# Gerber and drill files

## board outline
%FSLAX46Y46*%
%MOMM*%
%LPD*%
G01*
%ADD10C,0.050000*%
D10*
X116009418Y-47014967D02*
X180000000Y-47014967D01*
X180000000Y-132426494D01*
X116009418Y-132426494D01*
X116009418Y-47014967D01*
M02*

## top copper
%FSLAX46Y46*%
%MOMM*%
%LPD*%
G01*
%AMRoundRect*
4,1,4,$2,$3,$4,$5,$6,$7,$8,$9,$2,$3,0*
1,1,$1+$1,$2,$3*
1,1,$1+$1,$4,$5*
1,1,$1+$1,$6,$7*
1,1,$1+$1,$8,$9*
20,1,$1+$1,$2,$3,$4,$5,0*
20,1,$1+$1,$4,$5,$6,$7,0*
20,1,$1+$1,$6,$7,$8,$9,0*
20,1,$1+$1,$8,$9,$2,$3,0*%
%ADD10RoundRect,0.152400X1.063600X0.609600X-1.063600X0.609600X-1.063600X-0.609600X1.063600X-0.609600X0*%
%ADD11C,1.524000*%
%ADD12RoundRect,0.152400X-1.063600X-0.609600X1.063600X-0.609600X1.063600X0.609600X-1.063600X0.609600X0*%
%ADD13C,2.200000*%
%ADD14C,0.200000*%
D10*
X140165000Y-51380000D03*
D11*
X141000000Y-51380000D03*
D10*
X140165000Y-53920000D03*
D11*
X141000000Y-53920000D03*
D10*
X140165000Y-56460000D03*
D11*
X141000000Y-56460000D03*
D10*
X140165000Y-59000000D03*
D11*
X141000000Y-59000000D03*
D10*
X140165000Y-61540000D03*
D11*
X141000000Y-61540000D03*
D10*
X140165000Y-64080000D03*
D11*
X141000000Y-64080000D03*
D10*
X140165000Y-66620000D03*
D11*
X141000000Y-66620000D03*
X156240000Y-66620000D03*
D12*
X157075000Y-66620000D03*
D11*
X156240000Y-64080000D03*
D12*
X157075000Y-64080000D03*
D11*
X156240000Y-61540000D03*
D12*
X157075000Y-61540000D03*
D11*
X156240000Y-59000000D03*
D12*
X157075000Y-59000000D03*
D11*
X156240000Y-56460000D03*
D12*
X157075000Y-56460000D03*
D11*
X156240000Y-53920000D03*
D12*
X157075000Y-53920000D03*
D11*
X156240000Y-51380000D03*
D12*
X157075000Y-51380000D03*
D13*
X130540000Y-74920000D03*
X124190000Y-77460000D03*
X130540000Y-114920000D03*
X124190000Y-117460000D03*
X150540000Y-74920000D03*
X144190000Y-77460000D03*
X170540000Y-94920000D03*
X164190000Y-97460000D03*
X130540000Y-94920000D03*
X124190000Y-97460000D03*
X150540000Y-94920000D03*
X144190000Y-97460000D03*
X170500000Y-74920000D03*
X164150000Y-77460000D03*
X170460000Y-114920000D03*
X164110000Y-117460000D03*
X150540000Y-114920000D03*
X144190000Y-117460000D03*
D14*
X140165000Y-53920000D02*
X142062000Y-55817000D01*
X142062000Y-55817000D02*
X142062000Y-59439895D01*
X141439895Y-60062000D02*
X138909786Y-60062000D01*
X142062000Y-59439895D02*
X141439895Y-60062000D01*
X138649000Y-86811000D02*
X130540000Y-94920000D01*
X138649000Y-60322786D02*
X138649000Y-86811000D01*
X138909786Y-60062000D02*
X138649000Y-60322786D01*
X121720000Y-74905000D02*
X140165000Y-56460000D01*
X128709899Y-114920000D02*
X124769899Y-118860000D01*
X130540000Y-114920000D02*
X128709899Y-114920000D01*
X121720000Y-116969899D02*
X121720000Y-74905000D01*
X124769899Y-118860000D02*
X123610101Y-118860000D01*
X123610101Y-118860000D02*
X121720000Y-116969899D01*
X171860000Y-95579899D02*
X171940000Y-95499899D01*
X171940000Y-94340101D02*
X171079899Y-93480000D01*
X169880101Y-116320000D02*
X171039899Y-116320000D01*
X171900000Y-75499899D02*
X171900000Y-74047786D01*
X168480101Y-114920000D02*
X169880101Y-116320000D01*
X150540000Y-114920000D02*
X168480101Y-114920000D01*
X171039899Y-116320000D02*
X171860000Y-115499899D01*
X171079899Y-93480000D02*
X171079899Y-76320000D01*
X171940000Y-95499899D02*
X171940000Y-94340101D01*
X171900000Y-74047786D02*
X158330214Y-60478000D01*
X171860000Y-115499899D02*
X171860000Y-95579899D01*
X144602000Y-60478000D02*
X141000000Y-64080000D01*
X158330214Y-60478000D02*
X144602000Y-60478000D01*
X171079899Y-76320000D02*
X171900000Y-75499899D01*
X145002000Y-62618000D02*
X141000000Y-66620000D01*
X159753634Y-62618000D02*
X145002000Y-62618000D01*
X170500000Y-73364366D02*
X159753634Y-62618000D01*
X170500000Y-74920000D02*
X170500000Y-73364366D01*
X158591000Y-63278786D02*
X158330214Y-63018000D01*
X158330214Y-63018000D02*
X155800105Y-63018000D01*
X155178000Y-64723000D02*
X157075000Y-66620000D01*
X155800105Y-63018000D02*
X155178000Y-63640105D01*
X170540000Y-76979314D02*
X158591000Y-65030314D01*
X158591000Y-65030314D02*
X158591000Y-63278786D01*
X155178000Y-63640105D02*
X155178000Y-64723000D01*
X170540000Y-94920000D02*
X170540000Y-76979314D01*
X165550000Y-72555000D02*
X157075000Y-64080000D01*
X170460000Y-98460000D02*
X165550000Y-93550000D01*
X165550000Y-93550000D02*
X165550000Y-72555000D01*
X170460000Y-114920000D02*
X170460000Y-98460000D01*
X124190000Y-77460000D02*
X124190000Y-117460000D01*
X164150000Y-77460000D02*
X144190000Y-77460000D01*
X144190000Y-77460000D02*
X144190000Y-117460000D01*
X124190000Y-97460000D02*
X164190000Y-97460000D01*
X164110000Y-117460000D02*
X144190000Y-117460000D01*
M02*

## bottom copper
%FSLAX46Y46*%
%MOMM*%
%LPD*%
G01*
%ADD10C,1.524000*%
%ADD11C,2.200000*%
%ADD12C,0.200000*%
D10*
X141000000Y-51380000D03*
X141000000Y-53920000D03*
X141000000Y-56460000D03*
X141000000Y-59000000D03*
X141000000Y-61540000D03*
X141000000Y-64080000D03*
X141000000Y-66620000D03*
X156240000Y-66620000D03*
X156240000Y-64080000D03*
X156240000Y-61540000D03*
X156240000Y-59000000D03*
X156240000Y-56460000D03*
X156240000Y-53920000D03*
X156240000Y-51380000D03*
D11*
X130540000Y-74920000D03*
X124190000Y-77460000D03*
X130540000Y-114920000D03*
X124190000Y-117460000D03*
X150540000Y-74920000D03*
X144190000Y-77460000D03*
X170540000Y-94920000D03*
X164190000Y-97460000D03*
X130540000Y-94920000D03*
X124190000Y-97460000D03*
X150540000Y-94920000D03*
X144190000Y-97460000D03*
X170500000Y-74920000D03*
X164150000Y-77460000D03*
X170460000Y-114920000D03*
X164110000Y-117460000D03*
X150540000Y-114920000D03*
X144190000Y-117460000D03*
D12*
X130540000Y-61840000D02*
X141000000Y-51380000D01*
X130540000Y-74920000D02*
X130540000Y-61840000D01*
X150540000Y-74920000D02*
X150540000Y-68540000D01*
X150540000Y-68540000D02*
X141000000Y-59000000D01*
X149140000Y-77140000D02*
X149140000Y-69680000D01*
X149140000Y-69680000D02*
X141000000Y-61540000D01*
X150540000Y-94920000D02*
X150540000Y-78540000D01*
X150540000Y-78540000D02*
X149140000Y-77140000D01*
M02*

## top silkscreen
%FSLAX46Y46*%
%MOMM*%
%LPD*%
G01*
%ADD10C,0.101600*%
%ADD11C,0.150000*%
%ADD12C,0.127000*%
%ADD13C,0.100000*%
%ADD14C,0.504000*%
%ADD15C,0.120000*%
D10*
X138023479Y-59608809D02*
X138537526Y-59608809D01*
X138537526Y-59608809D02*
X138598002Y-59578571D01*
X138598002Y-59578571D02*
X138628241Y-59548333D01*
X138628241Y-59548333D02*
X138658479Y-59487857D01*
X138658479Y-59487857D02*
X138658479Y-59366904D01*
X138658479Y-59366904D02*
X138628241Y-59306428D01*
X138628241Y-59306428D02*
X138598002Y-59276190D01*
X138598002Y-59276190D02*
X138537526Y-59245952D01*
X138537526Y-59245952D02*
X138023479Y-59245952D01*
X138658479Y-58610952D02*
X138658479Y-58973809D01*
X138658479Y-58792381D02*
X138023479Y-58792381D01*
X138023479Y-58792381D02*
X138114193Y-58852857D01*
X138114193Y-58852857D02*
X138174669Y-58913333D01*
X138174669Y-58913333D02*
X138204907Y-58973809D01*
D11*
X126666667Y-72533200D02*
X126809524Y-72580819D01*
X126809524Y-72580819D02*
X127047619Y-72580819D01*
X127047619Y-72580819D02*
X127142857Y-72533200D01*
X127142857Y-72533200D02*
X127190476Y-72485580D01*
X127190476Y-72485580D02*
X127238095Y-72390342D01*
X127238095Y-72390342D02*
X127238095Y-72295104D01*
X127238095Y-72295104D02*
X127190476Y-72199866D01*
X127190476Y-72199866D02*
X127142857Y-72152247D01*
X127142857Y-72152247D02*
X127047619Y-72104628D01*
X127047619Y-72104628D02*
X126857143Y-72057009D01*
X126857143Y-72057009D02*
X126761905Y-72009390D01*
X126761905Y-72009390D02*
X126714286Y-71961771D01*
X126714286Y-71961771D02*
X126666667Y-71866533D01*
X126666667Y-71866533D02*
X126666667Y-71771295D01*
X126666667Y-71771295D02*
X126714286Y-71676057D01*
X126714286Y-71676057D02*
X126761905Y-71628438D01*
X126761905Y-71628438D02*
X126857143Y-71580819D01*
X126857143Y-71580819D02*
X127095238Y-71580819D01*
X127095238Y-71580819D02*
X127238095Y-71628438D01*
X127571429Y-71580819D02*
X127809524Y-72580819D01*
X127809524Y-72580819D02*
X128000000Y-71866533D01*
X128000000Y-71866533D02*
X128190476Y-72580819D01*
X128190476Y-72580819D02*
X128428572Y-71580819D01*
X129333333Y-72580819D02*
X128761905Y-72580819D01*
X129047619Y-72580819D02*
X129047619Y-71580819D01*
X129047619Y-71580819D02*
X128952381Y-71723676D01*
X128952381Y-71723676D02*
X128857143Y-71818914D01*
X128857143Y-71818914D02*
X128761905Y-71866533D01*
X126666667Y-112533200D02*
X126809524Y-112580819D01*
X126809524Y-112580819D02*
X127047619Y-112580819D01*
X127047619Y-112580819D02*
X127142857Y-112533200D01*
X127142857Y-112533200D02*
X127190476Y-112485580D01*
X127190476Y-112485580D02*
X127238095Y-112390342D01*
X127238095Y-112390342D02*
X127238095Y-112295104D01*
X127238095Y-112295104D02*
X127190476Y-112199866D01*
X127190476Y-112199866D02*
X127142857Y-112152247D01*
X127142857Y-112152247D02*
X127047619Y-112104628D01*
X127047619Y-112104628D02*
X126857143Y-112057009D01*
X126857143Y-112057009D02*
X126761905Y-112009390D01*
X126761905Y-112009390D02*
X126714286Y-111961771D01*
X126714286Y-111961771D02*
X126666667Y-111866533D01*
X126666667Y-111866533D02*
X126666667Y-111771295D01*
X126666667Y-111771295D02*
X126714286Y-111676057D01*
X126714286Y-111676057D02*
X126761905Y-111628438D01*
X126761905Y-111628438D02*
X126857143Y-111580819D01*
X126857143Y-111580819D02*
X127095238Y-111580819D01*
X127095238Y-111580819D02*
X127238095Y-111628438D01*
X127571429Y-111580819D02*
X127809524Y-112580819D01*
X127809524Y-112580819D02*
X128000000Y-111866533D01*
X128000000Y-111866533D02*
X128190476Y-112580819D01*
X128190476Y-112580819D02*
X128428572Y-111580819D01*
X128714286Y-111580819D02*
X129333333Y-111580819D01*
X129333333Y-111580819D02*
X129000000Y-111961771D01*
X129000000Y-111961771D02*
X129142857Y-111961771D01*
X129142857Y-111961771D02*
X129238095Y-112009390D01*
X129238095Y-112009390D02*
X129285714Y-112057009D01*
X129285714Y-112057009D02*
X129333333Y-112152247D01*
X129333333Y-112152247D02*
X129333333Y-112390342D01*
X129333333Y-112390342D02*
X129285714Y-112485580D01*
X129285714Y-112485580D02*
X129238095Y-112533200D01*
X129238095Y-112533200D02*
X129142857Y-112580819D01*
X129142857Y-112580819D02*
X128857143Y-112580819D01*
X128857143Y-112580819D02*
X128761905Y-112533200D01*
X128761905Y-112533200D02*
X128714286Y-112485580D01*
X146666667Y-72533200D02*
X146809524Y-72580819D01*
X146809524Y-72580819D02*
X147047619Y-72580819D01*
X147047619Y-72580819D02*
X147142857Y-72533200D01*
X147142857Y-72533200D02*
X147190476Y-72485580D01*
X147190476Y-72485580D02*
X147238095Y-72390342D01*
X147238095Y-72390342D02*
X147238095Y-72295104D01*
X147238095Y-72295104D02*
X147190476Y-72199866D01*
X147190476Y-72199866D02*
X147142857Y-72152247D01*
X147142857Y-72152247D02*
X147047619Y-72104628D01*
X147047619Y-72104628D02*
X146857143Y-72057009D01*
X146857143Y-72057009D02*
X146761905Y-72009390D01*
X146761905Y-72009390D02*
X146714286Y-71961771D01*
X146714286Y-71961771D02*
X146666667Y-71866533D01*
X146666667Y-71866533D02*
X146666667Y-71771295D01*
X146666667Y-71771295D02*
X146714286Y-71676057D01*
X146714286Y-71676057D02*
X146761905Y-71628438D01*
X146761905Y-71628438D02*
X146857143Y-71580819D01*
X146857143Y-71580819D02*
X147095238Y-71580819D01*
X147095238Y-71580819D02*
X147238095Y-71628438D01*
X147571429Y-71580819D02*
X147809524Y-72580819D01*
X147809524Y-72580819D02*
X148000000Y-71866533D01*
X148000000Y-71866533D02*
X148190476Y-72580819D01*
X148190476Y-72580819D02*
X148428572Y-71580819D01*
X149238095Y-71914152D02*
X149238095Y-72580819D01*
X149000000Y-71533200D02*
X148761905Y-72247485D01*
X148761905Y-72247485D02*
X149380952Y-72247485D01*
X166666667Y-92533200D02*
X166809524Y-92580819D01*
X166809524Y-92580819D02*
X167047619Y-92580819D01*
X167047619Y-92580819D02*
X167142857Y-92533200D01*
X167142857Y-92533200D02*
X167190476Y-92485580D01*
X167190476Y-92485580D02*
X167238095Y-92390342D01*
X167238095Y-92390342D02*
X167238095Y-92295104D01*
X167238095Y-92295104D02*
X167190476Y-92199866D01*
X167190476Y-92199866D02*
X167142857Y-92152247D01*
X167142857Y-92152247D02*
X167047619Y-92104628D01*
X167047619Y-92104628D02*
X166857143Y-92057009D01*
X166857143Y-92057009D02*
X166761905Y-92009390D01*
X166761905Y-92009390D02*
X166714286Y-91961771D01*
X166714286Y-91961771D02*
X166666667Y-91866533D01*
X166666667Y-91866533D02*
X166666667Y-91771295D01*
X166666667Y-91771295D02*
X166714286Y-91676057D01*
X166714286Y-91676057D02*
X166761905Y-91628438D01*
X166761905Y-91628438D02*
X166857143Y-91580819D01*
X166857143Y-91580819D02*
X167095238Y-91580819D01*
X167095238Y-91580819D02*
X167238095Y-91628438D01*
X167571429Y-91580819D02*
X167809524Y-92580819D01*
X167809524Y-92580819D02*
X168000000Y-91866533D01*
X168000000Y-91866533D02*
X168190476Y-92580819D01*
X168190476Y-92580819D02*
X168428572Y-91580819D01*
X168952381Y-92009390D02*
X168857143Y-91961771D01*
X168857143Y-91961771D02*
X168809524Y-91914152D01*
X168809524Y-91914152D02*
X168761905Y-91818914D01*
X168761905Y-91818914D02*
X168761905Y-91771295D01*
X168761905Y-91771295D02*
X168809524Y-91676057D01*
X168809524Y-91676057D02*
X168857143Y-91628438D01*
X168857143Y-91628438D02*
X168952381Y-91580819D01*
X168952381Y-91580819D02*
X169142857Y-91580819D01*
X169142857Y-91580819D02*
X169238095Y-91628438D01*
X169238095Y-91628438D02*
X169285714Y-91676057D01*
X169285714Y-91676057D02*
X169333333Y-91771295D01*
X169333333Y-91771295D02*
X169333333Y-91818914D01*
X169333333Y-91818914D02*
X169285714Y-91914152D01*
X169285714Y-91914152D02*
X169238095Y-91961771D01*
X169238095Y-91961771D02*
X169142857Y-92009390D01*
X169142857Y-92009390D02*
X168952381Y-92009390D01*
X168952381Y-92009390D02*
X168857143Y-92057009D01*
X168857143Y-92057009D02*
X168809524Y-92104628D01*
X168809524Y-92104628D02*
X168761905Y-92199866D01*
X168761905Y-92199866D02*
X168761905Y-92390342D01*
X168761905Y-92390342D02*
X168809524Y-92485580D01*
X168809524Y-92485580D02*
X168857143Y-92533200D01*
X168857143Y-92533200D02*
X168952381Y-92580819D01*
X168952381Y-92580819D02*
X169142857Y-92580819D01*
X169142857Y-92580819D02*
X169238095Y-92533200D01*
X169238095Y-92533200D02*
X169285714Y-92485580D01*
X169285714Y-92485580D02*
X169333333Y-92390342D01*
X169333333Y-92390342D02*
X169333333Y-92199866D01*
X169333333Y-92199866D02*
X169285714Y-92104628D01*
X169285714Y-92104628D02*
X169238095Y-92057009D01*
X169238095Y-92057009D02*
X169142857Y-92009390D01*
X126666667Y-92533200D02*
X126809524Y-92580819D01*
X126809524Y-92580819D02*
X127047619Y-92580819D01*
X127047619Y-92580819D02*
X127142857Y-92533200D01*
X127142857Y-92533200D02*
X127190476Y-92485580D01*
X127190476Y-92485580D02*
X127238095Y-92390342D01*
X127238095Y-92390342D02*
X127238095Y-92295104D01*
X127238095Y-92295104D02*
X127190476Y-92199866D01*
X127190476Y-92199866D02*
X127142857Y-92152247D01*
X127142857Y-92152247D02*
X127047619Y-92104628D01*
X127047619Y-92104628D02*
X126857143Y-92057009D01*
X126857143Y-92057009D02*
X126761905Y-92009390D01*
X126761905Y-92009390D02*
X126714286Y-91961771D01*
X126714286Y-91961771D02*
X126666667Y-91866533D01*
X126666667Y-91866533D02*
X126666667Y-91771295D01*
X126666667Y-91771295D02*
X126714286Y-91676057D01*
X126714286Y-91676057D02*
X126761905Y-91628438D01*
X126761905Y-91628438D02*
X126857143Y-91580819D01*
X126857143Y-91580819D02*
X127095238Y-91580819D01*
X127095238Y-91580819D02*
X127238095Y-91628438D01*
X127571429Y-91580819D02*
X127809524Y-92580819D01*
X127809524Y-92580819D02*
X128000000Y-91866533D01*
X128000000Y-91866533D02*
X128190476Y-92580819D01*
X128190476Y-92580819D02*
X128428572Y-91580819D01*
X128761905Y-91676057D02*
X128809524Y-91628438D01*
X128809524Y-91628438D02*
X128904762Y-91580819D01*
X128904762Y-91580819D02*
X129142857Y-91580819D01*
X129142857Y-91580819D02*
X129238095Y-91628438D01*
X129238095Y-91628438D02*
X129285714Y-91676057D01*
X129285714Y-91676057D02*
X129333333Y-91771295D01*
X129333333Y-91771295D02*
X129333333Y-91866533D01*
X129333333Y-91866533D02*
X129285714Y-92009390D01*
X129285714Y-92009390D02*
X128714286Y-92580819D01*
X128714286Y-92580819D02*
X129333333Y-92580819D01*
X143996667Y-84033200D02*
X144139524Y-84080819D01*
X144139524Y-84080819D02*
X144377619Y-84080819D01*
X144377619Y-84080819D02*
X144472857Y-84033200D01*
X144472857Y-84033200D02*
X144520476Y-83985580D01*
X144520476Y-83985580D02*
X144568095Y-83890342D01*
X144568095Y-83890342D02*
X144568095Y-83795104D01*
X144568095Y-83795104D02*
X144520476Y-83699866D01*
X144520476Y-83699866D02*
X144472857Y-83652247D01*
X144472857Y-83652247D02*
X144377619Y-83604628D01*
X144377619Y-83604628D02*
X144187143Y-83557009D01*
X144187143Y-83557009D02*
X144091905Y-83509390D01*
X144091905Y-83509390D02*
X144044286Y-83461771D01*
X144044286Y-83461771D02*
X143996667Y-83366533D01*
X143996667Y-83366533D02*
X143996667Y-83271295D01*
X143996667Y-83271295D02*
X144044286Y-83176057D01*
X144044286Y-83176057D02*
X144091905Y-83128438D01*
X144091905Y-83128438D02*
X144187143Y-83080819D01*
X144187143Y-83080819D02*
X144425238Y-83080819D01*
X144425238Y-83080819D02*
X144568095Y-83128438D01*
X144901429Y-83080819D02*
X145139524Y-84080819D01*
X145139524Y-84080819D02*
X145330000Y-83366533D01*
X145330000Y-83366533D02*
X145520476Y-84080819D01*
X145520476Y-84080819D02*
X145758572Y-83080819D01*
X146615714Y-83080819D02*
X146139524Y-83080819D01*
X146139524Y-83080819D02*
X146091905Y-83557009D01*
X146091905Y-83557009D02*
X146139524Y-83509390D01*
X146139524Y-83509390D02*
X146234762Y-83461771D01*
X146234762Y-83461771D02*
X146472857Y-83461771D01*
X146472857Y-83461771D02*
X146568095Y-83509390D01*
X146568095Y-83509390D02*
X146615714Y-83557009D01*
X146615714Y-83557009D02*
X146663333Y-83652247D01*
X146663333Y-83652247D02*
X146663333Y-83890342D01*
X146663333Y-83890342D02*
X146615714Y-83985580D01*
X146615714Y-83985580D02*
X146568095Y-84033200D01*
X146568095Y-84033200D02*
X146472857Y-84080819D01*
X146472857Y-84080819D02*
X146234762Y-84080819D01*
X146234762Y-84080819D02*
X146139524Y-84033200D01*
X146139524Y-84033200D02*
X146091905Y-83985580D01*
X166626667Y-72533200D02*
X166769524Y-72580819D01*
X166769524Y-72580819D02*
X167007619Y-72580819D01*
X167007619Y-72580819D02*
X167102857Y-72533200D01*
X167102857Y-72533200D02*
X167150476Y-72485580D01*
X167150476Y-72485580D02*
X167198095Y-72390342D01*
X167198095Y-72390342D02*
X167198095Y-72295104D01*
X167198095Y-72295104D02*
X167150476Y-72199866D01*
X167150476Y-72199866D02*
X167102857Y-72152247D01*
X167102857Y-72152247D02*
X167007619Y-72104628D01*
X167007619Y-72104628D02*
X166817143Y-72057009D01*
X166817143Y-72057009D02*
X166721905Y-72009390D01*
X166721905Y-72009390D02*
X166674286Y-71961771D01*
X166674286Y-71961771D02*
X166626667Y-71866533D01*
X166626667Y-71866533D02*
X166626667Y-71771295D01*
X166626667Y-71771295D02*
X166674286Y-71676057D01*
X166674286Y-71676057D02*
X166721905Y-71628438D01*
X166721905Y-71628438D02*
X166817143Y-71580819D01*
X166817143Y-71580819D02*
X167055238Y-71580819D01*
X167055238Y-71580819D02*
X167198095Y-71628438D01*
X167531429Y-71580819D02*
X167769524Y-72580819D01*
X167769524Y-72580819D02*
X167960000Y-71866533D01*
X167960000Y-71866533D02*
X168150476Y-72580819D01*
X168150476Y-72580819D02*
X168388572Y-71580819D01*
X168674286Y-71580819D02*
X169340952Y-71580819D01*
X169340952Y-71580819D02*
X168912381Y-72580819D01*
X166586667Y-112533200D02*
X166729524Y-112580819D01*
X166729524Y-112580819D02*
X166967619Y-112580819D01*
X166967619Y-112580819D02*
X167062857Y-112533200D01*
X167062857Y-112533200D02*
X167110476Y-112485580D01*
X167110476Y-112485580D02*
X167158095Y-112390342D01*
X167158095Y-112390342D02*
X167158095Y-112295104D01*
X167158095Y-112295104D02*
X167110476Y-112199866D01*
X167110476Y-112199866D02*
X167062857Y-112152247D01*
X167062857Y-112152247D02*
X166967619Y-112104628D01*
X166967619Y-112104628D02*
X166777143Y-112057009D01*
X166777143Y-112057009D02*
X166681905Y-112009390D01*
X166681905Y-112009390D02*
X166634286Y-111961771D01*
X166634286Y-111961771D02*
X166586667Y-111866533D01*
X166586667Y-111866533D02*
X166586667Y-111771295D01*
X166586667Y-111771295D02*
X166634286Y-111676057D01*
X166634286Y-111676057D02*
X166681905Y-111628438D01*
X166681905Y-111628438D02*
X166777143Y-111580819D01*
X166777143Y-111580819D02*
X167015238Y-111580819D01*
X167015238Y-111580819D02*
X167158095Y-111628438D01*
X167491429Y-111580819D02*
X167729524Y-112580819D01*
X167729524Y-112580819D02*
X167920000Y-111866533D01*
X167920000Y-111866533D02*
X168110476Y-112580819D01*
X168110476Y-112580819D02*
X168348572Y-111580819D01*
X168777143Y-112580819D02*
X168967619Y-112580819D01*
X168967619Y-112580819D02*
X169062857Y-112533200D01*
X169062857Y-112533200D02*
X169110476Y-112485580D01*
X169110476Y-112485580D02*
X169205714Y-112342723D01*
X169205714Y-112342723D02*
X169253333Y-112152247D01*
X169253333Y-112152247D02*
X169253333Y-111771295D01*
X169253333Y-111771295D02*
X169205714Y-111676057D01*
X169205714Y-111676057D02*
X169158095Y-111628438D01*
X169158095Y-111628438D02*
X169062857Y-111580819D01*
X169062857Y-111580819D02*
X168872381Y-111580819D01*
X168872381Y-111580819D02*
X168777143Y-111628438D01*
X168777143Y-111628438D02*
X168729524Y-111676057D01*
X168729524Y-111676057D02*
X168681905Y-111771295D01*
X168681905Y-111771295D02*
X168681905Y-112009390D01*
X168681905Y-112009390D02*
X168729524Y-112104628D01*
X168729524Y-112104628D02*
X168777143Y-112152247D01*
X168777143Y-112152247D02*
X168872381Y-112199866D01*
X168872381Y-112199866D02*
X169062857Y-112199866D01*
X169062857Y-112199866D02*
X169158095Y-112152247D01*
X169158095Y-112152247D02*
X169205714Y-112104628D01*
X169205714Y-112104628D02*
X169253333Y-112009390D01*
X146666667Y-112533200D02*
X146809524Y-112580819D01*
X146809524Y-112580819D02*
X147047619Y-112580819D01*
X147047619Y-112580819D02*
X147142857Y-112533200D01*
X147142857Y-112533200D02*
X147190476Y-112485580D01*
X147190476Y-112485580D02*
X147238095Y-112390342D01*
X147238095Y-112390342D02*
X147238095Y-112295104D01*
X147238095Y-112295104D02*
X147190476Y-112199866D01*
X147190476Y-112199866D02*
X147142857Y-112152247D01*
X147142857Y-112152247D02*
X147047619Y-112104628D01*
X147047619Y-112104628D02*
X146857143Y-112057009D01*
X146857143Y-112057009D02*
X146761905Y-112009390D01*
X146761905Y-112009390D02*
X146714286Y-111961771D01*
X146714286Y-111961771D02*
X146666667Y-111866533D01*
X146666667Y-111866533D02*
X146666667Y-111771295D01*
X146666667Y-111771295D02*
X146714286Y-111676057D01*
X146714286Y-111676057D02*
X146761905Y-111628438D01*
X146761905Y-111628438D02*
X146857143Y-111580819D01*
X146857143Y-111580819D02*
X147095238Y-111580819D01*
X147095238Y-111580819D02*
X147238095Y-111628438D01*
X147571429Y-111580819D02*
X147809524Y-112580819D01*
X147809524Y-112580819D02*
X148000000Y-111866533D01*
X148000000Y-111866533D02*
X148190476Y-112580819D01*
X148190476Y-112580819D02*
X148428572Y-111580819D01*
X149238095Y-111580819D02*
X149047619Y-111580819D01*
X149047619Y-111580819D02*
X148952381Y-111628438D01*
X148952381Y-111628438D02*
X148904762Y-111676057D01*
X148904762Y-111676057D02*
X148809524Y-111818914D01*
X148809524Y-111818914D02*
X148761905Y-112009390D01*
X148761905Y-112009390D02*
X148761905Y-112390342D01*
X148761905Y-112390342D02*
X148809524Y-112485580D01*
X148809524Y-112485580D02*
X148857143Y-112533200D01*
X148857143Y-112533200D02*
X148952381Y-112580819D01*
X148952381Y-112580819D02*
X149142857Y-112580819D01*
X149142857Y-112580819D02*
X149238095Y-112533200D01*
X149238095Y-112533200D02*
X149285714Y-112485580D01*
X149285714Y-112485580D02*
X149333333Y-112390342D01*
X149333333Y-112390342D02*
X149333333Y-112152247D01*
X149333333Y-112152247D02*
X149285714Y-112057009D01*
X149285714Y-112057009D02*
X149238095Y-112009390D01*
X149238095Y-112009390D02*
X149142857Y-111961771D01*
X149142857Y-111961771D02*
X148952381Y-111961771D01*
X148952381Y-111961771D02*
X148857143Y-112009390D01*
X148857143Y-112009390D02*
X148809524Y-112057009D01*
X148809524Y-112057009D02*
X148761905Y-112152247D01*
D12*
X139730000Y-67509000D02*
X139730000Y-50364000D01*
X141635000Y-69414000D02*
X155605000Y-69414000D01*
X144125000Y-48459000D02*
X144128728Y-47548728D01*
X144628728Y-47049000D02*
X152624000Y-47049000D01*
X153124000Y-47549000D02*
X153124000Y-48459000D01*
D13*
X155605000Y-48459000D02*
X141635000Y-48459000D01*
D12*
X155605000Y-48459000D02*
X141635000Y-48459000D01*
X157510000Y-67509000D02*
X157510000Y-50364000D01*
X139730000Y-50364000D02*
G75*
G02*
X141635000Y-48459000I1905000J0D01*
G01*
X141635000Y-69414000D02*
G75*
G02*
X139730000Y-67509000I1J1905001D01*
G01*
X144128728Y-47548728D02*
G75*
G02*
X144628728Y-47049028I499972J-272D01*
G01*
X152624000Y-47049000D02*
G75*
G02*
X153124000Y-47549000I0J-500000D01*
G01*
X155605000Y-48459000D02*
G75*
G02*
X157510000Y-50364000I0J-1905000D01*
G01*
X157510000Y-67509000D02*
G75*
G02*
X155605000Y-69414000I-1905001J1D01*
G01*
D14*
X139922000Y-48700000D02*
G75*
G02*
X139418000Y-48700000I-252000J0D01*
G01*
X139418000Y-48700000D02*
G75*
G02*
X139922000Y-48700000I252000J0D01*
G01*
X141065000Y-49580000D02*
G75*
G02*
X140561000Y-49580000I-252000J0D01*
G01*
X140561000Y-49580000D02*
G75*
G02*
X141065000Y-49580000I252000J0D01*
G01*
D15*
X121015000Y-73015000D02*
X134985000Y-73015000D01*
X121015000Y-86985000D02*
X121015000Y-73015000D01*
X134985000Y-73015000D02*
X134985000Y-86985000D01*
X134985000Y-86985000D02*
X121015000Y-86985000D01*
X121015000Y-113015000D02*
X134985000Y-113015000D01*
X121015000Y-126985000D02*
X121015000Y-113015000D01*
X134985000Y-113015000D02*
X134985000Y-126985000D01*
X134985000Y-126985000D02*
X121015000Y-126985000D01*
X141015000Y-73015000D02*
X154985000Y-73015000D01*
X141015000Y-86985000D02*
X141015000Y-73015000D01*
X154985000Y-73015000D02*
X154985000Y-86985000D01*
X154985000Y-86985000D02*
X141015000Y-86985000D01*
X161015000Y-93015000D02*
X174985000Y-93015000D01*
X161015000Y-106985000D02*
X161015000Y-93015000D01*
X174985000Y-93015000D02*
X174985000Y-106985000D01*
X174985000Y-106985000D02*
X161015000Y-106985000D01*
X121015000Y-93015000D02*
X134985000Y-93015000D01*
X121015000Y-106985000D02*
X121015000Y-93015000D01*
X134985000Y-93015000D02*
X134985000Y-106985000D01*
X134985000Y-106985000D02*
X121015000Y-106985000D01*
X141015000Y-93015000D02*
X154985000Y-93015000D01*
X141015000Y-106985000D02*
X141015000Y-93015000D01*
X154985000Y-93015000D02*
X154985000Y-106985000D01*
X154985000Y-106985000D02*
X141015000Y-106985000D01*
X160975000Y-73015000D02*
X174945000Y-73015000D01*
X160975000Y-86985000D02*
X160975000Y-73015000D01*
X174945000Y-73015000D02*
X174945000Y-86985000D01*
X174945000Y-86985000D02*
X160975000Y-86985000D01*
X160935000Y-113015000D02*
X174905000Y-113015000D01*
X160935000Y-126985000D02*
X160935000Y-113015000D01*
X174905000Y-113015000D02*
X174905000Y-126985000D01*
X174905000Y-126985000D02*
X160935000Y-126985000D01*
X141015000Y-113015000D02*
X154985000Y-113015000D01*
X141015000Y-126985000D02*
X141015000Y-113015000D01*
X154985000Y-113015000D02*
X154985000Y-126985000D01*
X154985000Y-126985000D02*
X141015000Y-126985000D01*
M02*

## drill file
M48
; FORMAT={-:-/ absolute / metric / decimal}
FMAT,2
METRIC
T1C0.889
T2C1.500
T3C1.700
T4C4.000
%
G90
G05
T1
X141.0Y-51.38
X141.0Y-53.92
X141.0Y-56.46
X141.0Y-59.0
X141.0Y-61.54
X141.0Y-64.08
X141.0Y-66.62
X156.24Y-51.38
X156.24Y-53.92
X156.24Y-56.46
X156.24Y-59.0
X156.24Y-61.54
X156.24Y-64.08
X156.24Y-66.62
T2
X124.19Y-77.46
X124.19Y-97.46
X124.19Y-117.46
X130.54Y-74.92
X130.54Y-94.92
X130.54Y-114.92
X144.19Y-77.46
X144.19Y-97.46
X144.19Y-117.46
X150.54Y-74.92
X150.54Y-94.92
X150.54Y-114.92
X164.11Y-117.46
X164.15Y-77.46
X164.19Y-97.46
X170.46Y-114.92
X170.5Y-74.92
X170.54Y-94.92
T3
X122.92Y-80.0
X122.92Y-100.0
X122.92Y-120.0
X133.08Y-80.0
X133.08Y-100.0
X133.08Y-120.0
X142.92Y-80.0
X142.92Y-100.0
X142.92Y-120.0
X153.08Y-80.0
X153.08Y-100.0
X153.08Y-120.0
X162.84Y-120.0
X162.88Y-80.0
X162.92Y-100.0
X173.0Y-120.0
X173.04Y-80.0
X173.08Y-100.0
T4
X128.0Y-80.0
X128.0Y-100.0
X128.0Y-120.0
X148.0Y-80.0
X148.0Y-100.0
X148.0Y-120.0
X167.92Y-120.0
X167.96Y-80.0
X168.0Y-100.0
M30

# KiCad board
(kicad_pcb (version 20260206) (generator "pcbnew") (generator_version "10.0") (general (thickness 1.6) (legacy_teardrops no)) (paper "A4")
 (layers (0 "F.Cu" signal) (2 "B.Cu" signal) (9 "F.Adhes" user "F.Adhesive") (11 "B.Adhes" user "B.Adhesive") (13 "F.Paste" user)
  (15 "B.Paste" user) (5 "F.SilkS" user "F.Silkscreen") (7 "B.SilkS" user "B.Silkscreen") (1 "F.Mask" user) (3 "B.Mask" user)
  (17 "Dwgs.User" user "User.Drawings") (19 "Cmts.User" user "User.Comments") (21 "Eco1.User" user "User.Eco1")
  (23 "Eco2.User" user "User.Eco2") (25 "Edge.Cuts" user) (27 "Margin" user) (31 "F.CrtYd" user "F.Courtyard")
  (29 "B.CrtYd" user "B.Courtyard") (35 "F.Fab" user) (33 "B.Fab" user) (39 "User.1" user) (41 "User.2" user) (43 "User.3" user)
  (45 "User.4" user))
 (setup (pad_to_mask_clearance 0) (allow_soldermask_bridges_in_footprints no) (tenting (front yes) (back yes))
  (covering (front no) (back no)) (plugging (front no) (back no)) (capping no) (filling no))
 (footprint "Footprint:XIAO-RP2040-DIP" (layer "F.Cu") (at 148.62 59 90)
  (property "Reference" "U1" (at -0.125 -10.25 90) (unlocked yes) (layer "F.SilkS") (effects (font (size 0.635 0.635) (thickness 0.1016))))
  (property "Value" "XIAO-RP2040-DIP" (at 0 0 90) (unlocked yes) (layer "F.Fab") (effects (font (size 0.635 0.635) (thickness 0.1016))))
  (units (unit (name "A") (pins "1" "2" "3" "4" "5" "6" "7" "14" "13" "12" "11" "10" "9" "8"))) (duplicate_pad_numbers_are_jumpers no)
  (fp_line (start -8.509 -8.89) (end 8.636 -8.89) (stroke (width 0.127) (type solid)) (layer "F.SilkS"))
  (fp_line (start -10.414 -6.985) (end -10.414 6.985) (stroke (width 0.127) (type solid)) (layer "F.SilkS"))
  (fp_line (start 10.541 -4.495) (end 11.451272 -4.491272) (stroke (width 0.127) (type solid)) (layer "F.SilkS"))
  (fp_line (start 11.951 -3.991272) (end 11.951 4.004) (stroke (width 0.127) (type solid)) (layer "F.SilkS"))
  (fp_line (start 11.451 4.504) (end 10.541 4.504) (stroke (width 0.127) (type solid)) (layer "F.SilkS"))
  (fp_line (start 10.541 6.985) (end 10.541 -6.985) (stroke (width 0.1) (type solid)) (layer "F.SilkS"))
  (fp_line (start 10.541 6.985) (end 10.541 -6.985) (stroke (width 0.127) (type solid)) (layer "F.SilkS"))
  (fp_line (start -8.509 8.89) (end 8.636 8.89) (stroke (width 0.127) (type solid)) (layer "F.SilkS"))
  (fp_arc (start 8.636 -8.89) (mid 9.983038 -8.332038) (end 10.541 -6.985) (stroke (width 0.127) (type solid)) (layer "F.SilkS"))
  (fp_arc (start -10.414 -6.985) (mid -9.856038 -8.332038) (end -8.509 -8.89) (stroke (width 0.127) (type solid)) (layer "F.SilkS"))
  (fp_arc (start 11.451272 -4.491272) (mid 11.804644 -4.344724) (end 11.951 -3.991272) (stroke (width 0.127) (type default))
   (layer "F.SilkS"))
  (fp_arc (start 11.951 4.004) (mid 11.804553 4.357553) (end 11.451 4.504) (stroke (width 0.127) (type default)) (layer "F.SilkS"))
  (fp_arc (start 10.541 6.985) (mid 9.983038 8.332038) (end 8.636 8.89) (stroke (width 0.127) (type solid)) (layer "F.SilkS"))
  (fp_arc (start -8.509 8.89) (mid -9.856038 8.332038) (end -10.414 6.985) (stroke (width 0.127) (type solid)) (layer "F.SilkS"))
  (fp_circle (center 10.3 -8.95) (end 10.554 -8.95) (stroke (width 0.5) (type solid)) (fill yes) (layer "F.SilkS"))
  (fp_circle (center 9.42 -7.807) (end 9.674 -7.807) (stroke (width 0.5) (type solid)) (fill yes) (layer "F.SilkS"))
  (pad "1" smd roundrect (at 7.62 -8.455 180) (size 2.432 1.524) (layers "F.Cu" "F.Mask") (roundrect_rratio 0.1) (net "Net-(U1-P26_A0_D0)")
   (thermal_bridge_angle 45))
  (pad "1" thru_hole circle (at 7.62 -7.62 180) (size 1.524 1.524) (drill 0.889) (layers "*.Cu" "*.Mask") (remove_unused_layers no)
   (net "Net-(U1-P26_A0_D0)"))
  (pad "2" smd roundrect (at 5.08 -8.455 180) (size 2.432 1.524) (layers "F.Cu" "F.Mask") (roundrect_rratio 0.1) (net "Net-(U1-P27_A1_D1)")
   (thermal_bridge_angle 45))
  (pad "2" thru_hole circle (at 5.08 -7.62 180) (size 1.524 1.524) (drill 0.889) (layers "*.Cu" "*.Mask") (remove_unused_layers no)
   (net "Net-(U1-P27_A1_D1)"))
  (pad "3" smd roundrect (at 2.54 -8.455 180) (size 2.432 1.524) (layers "F.Cu" "F.Mask") (roundrect_rratio 0.1) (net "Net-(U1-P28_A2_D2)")
   (thermal_bridge_angle 45))
  (pad "3" thru_hole circle (at 2.54 -7.62 180) (size 1.524 1.524) (drill 0.889) (layers "*.Cu" "*.Mask") (remove_unused_layers no)
   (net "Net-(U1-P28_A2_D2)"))
  (pad "4" smd roundrect (at 0 -8.455 180) (size 2.432 1.524) (layers "F.Cu" "F.Mask") (roundrect_rratio 0.1) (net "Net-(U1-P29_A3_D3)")
   (thermal_bridge_angle 45))
  (pad "4" thru_hole circle (at 0 -7.62 180) (size 1.524 1.524) (drill 0.889) (layers "*.Cu" "*.Mask") (remove_unused_layers no)
   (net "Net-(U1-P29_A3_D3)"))
  (pad "5" smd roundrect (at -2.54 -8.455 180) (size 2.432 1.524) (layers "F.Cu" "F.Mask") (roundrect_rratio 0.1) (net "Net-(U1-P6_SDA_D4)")
   (thermal_bridge_angle 45))
  (pad "5" thru_hole circle (at -2.54 -7.62 180) (size 1.524 1.524) (drill 0.889) (layers "*.Cu" "*.Mask") (remove_unused_layers no)
   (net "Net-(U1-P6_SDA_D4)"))
  (pad "6" smd roundrect (at -5.08 -8.455 180) (size 2.432 1.524) (layers "F.Cu" "F.Mask") (roundrect_rratio 0.1) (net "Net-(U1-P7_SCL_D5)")
   (thermal_bridge_angle 45))
  (pad "6" thru_hole circle (at -5.08 -7.62 180) (size 1.524 1.524) (drill 0.889) (layers "*.Cu" "*.Mask") (remove_unused_layers no)
   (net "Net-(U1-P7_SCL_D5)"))
  (pad "7" smd roundrect (at -7.62 -8.455 180) (size 2.432 1.524) (layers "F.Cu" "F.Mask") (roundrect_rratio 0.1) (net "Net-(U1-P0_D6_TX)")
   (thermal_bridge_angle 45))
  (pad "7" thru_hole circle (at -7.62 -7.62 180) (size 1.524 1.524) (drill 0.889) (layers "*.Cu" "*.Mask") (remove_unused_layers no)
   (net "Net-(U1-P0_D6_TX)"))
  (pad "8" thru_hole circle (at -7.62 7.62) (size 1.524 1.524) (drill 0.889) (layers "*.Cu" "*.Mask") (remove_unused_layers no)
   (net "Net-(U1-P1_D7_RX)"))
  (pad "8" smd roundrect (at -7.62 8.455) (size 2.432 1.524) (layers "F.Cu" "F.Mask") (roundrect_rratio 0.1) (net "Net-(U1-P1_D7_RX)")
   (thermal_bridge_angle 45))
  (pad "9" thru_hole circle (at -5.08 7.62) (size 1.524 1.524) (drill 0.889) (layers "*.Cu" "*.Mask") (remove_unused_layers no)
   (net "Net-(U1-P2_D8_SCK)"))
  (pad "9" smd roundrect (at -5.08 8.455) (size 2.432 1.524) (layers "F.Cu" "F.Mask") (roundrect_rratio 0.1) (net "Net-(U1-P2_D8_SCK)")
   (thermal_bridge_angle 45))
  (pad "10" thru_hole circle (at -2.54 7.62) (size 1.524 1.524) (drill 0.889) (layers "*.Cu" "*.Mask") (remove_unused_layers no)
   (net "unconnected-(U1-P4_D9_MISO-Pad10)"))
  (pad "10" smd roundrect (at -2.54 8.455) (size 2.432 1.524) (layers "F.Cu" "F.Mask") (roundrect_rratio 0.1)
   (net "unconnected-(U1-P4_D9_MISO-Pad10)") (thermal_bridge_angle 45))
  (pad "11" thru_hole circle (at 0 7.62) (size 1.524 1.524) (drill 0.889) (layers "*.Cu" "*.Mask") (remove_unused_layers no)
   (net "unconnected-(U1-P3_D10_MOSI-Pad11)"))
  (pad "11" smd roundrect (at 0 8.455) (size 2.432 1.524) (layers "F.Cu" "F.Mask") (roundrect_rratio 0.1)
   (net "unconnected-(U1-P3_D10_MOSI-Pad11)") (thermal_bridge_angle 45))
  (pad "12" thru_hole circle (at 2.54 7.62) (size 1.524 1.524) (drill 0.889) (layers "*.Cu" "*.Mask") (remove_unused_layers no)
   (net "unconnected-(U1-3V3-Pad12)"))
  (pad "12" smd roundrect (at 2.54 8.455) (size 2.432 1.524) (layers "F.Cu" "F.Mask") (roundrect_rratio 0.1)
   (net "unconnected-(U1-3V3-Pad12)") (thermal_bridge_angle 45))
  (pad "13" thru_hole circle (at 5.08 7.62) (size 1.524 1.524) (drill 0.889) (layers "*.Cu" "*.Mask") (remove_unused_layers no)
   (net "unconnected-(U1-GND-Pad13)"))
  (pad "13" smd roundrect (at 5.08 8.455) (size 2.432 1.524) (layers "F.Cu" "F.Mask") (roundrect_rratio 0.1)
   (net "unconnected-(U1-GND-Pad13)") (thermal_bridge_angle 45))
  (pad "14" thru_hole circle (at 7.62 7.62) (size 1.524 1.524) (drill 0.889) (layers "*.Cu" "*.Mask") (remove_unused_layers no)
   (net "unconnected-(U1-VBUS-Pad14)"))
  (pad "14" smd roundrect (at 7.62 8.455) (size 2.432 1.524) (layers "F.Cu" "F.Mask") (roundrect_rratio 0.1)
   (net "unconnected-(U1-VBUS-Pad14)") (thermal_bridge_angle 45)))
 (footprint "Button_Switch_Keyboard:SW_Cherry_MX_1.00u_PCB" (layer "F.Cu") (at 130.54 74.92)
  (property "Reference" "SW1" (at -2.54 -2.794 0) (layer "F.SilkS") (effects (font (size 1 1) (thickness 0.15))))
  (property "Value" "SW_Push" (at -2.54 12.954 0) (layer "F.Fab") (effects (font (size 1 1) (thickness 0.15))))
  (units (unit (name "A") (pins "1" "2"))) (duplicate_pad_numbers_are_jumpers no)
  (fp_line (start -9.525 -1.905) (end 4.445 -1.905) (stroke (width 0.12) (type solid)) (layer "F.SilkS"))
  (fp_line (start -9.525 12.065) (end -9.525 -1.905) (stroke (width 0.12) (type solid)) (layer "F.SilkS"))
  (fp_line (start 4.445 -1.905) (end 4.445 12.065) (stroke (width 0.12) (type solid)) (layer "F.SilkS"))
  (fp_line (start 4.445 12.065) (end -9.525 12.065) (stroke (width 0.12) (type solid)) (layer "F.SilkS"))
  (pad "" np_thru_hole circle (at -7.62 5.08) (size 1.7 1.7) (drill 1.7) (layers "*.Cu" "*.Mask"))
  (pad "" np_thru_hole circle (at -2.54 5.08) (size 4 4) (drill 4) (layers "*.Cu" "*.Mask"))
  (pad "" np_thru_hole circle (at 2.54 5.08) (size 1.7 1.7) (drill 1.7) (layers "*.Cu" "*.Mask"))
  (pad "1" thru_hole circle (at 0 0) (size 2.2 2.2) (drill 1.5) (layers "*.Cu" "*.Mask") (remove_unused_layers no)
   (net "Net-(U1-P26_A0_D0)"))
  (pad "2" thru_hole circle (at -6.35 2.54) (size 2.2 2.2) (drill 1.5) (layers "*.Cu" "*.Mask") (remove_unused_layers no) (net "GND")))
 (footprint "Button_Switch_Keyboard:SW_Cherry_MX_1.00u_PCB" (layer "F.Cu") (at 130.54 114.92)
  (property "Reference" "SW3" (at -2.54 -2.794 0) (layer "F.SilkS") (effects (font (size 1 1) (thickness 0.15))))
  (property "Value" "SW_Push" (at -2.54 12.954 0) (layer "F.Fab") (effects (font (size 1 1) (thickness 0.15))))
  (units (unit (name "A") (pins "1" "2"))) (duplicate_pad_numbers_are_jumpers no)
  (fp_line (start -9.525 -1.905) (end 4.445 -1.905) (stroke (width 0.12) (type solid)) (layer "F.SilkS"))
  (fp_line (start -9.525 12.065) (end -9.525 -1.905) (stroke (width 0.12) (type solid)) (layer "F.SilkS"))
  (fp_line (start 4.445 -1.905) (end 4.445 12.065) (stroke (width 0.12) (type solid)) (layer "F.SilkS"))
  (fp_line (start 4.445 12.065) (end -9.525 12.065) (stroke (width 0.12) (type solid)) (layer "F.SilkS"))
  (pad "" np_thru_hole circle (at -7.62 5.08) (size 1.7 1.7) (drill 1.7) (layers "*.Cu" "*.Mask"))
  (pad "" np_thru_hole circle (at -2.54 5.08) (size 4 4) (drill 4) (layers "*.Cu" "*.Mask"))
  (pad "" np_thru_hole circle (at 2.54 5.08) (size 1.7 1.7) (drill 1.7) (layers "*.Cu" "*.Mask"))
  (pad "1" thru_hole circle (at 0 0) (size 2.2 2.2) (drill 1.5) (layers "*.Cu" "*.Mask") (remove_unused_layers no)
   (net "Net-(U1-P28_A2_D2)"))
  (pad "2" thru_hole circle (at -6.35 2.54) (size 2.2 2.2) (drill 1.5) (layers "*.Cu" "*.Mask") (remove_unused_layers no) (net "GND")))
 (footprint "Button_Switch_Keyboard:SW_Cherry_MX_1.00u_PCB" (layer "F.Cu") (at 150.54 74.92)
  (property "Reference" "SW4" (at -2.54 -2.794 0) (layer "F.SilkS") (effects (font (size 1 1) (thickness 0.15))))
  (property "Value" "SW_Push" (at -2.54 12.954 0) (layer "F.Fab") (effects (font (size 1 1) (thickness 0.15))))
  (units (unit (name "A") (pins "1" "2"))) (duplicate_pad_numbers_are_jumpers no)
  (fp_line (start -9.525 -1.905) (end 4.445 -1.905) (stroke (width 0.12) (type solid)) (layer "F.SilkS"))
  (fp_line (start -9.525 12.065) (end -9.525 -1.905) (stroke (width 0.12) (type solid)) (layer "F.SilkS"))
  (fp_line (start 4.445 -1.905) (end 4.445 12.065) (stroke (width 0.12) (type solid)) (layer "F.SilkS"))
  (fp_line (start 4.445 12.065) (end -9.525 12.065) (stroke (width 0.12) (type solid)) (layer "F.SilkS"))
  (pad "" np_thru_hole circle (at -7.62 5.08) (size 1.7 1.7) (drill 1.7) (layers "*.Cu" "*.Mask"))
  (pad "" np_thru_hole circle (at -2.54 5.08) (size 4 4) (drill 4) (layers "*.Cu" "*.Mask"))
  (pad "" np_thru_hole circle (at 2.54 5.08) (size 1.7 1.7) (drill 1.7) (layers "*.Cu" "*.Mask"))
  (pad "1" thru_hole circle (at 0 0) (size 2.2 2.2) (drill 1.5) (layers "*.Cu" "*.Mask") (remove_unused_layers no)
   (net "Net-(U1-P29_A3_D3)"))
  (pad "2" thru_hole circle (at -6.35 2.54) (size 2.2 2.2) (drill 1.5) (layers "*.Cu" "*.Mask") (remove_unused_layers no) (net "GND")))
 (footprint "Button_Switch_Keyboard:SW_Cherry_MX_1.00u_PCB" (layer "F.Cu") (at 170.54 94.92)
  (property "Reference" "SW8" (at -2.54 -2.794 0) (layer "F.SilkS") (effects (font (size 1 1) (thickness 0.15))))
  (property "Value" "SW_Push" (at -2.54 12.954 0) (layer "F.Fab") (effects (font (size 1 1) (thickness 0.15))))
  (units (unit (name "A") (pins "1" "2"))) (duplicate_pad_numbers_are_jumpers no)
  (fp_line (start -9.525 -1.905) (end 4.445 -1.905) (stroke (width 0.12) (type solid)) (layer "F.SilkS"))
  (fp_line (start -9.525 12.065) (end -9.525 -1.905) (stroke (width 0.12) (type solid)) (layer "F.SilkS"))
  (fp_line (start 4.445 -1.905) (end 4.445 12.065) (stroke (width 0.12) (type solid)) (layer "F.SilkS"))
  (fp_line (start 4.445 12.065) (end -9.525 12.065) (stroke (width 0.12) (type solid)) (layer "F.SilkS"))
  (pad "" np_thru_hole circle (at -7.62 5.08) (size 1.7 1.7) (drill 1.7) (layers "*.Cu" "*.Mask"))
  (pad "" np_thru_hole circle (at -2.54 5.08) (size 4 4) (drill 4) (layers "*.Cu" "*.Mask"))
  (pad "" np_thru_hole circle (at 2.54 5.08) (size 1.7 1.7) (drill 1.7) (layers "*.Cu" "*.Mask"))
  (pad "1" thru_hole circle (at 0 0) (size 2.2 2.2) (drill 1.5) (layers "*.Cu" "*.Mask") (remove_unused_layers no) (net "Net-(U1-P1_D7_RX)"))
  (pad "2" thru_hole circle (at -6.35 2.54) (size 2.2 2.2) (drill 1.5) (layers "*.Cu" "*.Mask") (remove_unused_layers no) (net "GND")))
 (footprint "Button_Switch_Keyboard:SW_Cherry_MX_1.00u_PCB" (layer "F.Cu") (at 130.54 94.92)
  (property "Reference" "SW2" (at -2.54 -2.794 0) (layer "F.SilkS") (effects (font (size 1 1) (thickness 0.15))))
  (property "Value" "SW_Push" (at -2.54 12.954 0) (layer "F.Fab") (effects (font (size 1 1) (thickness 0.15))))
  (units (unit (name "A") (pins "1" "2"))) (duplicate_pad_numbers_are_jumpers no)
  (fp_line (start -9.525 -1.905) (end 4.445 -1.905) (stroke (width 0.12) (type solid)) (layer "F.SilkS"))
  (fp_line (start -9.525 12.065) (end -9.525 -1.905) (stroke (width 0.12) (type solid)) (layer "F.SilkS"))
  (fp_line (start 4.445 -1.905) (end 4.445 12.065) (stroke (width 0.12) (type solid)) (layer "F.SilkS"))
  (fp_line (start 4.445 12.065) (end -9.525 12.065) (stroke (width 0.12) (type solid)) (layer "F.SilkS"))
  (pad "" np_thru_hole circle (at -7.62 5.08) (size 1.7 1.7) (drill 1.7) (layers "*.Cu" "*.Mask"))
  (pad "" np_thru_hole circle (at -2.54 5.08) (size 4 4) (drill 4) (layers "*.Cu" "*.Mask"))
  (pad "" np_thru_hole circle (at 2.54 5.08) (size 1.7 1.7) (drill 1.7) (layers "*.Cu" "*.Mask"))
  (pad "1" thru_hole circle (at 0 0) (size 2.2 2.2) (drill 1.5) (layers "*.Cu" "*.Mask") (remove_unused_layers no)
   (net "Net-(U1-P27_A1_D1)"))
  (pad "2" thru_hole circle (at -6.35 2.54) (size 2.2 2.2) (drill 1.5) (layers "*.Cu" "*.Mask") (remove_unused_layers no) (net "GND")))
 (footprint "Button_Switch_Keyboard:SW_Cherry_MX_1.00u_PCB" (layer "F.Cu") (at 150.54 94.92)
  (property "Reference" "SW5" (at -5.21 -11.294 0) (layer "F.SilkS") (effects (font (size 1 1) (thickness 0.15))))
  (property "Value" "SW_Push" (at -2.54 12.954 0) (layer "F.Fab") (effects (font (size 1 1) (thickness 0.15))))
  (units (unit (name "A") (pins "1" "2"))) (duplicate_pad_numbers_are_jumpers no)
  (fp_line (start -9.525 -1.905) (end 4.445 -1.905) (stroke (width 0.12) (type solid)) (layer "F.SilkS"))
  (fp_line (start -9.525 12.065) (end -9.525 -1.905) (stroke (width 0.12) (type solid)) (layer "F.SilkS"))
  (fp_line (start 4.445 -1.905) (end 4.445 12.065) (stroke (width 0.12) (type solid)) (layer "F.SilkS"))
  (fp_line (start 4.445 12.065) (end -9.525 12.065) (stroke (width 0.12) (type solid)) (layer "F.SilkS"))
  (pad "" np_thru_hole circle (at -7.62 5.08) (size 1.7 1.7) (drill 1.7) (layers "*.Cu" "*.Mask"))
  (pad "" np_thru_hole circle (at -2.54 5.08) (size 4 4) (drill 4) (layers "*.Cu" "*.Mask"))
  (pad "" np_thru_hole circle (at 2.54 5.08) (size 1.7 1.7) (drill 1.7) (layers "*.Cu" "*.Mask"))
  (pad "1" thru_hole circle (at 0 0) (size 2.2 2.2) (drill 1.5) (layers "*.Cu" "*.Mask") (remove_unused_layers no)
   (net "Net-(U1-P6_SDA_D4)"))
  (pad "2" thru_hole circle (at -6.35 2.54) (size 2.2 2.2) (drill 1.5) (layers "*.Cu" "*.Mask") (remove_unused_layers no) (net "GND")))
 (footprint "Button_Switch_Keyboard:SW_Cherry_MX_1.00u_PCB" (layer "F.Cu") (at 170.5 74.92)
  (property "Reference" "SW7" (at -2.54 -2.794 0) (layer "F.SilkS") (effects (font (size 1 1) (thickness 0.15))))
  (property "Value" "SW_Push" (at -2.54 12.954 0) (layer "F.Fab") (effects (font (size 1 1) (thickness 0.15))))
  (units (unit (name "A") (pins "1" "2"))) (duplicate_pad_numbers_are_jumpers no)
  (fp_line (start -9.525 -1.905) (end 4.445 -1.905) (stroke (width 0.12) (type solid)) (layer "F.SilkS"))
  (fp_line (start -9.525 12.065) (end -9.525 -1.905) (stroke (width 0.12) (type solid)) (layer "F.SilkS"))
  (fp_line (start 4.445 -1.905) (end 4.445 12.065) (stroke (width 0.12) (type solid)) (layer "F.SilkS"))
  (fp_line (start 4.445 12.065) (end -9.525 12.065) (stroke (width 0.12) (type solid)) (layer "F.SilkS"))
  (pad "" np_thru_hole circle (at -7.62 5.08) (size 1.7 1.7) (drill 1.7) (layers "*.Cu" "*.Mask"))
  (pad "" np_thru_hole circle (at -2.54 5.08) (size 4 4) (drill 4) (layers "*.Cu" "*.Mask"))
  (pad "" np_thru_hole circle (at 2.54 5.08) (size 1.7 1.7) (drill 1.7) (layers "*.Cu" "*.Mask"))
  (pad "1" thru_hole circle (at 0 0) (size 2.2 2.2) (drill 1.5) (layers "*.Cu" "*.Mask") (remove_unused_layers no) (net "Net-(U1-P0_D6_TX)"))
  (pad "2" thru_hole circle (at -6.35 2.54) (size 2.2 2.2) (drill 1.5) (layers "*.Cu" "*.Mask") (remove_unused_layers no) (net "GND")))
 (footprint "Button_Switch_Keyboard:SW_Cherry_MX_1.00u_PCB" (layer "F.Cu") (at 170.46 114.92)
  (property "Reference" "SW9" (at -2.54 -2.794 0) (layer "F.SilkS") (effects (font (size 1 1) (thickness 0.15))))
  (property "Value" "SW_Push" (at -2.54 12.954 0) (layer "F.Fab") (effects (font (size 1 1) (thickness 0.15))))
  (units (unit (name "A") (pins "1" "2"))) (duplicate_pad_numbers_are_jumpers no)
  (fp_line (start -9.525 -1.905) (end 4.445 -1.905) (stroke (width 0.12) (type solid)) (layer "F.SilkS"))
  (fp_line (start -9.525 12.065) (end -9.525 -1.905) (stroke (width 0.12) (type solid)) (layer "F.SilkS"))
  (fp_line (start 4.445 -1.905) (end 4.445 12.065) (stroke (width 0.12) (type solid)) (layer "F.SilkS"))
  (fp_line (start 4.445 12.065) (end -9.525 12.065) (stroke (width 0.12) (type solid)) (layer "F.SilkS"))
  (pad "" np_thru_hole circle (at -7.62 5.08) (size 1.7 1.7) (drill 1.7) (layers "*.Cu" "*.Mask"))
  (pad "" np_thru_hole circle (at -2.54 5.08) (size 4 4) (drill 4) (layers "*.Cu" "*.Mask"))
  (pad "" np_thru_hole circle (at 2.54 5.08) (size 1.7 1.7) (drill 1.7) (layers "*.Cu" "*.Mask"))
  (pad "1" thru_hole circle (at 0 0) (size 2.2 2.2) (drill 1.5) (layers "*.Cu" "*.Mask") (remove_unused_layers no)
   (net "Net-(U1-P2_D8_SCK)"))
  (pad "2" thru_hole circle (at -6.35 2.54) (size 2.2 2.2) (drill 1.5) (layers "*.Cu" "*.Mask") (remove_unused_layers no) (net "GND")))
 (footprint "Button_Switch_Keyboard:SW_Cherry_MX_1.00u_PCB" (layer "F.Cu") (at 150.54 114.92)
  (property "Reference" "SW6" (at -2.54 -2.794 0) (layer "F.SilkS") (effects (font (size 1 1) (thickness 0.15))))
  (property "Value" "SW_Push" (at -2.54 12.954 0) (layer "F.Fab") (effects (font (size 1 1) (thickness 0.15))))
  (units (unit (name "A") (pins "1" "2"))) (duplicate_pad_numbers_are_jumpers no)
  (fp_line (start -9.525 -1.905) (end 4.445 -1.905) (stroke (width 0.12) (type solid)) (layer "F.SilkS"))
  (fp_line (start -9.525 12.065) (end -9.525 -1.905) (stroke (width 0.12) (type solid)) (layer "F.SilkS"))
  (fp_line (start 4.445 -1.905) (end 4.445 12.065) (stroke (width 0.12) (type solid)) (layer "F.SilkS"))
  (fp_line (start 4.445 12.065) (end -9.525 12.065) (stroke (width 0.12) (type solid)) (layer "F.SilkS"))
  (pad "" np_thru_hole circle (at -7.62 5.08) (size 1.7 1.7) (drill 1.7) (layers "*.Cu" "*.Mask"))
  (pad "" np_thru_hole circle (at -2.54 5.08) (size 4 4) (drill 4) (layers "*.Cu" "*.Mask"))
  (pad "" np_thru_hole circle (at 2.54 5.08) (size 1.7 1.7) (drill 1.7) (layers "*.Cu" "*.Mask"))
  (pad "1" thru_hole circle (at 0 0) (size 2.2 2.2) (drill 1.5) (layers "*.Cu" "*.Mask") (remove_unused_layers no)
   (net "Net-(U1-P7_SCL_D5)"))
  (pad "2" thru_hole circle (at -6.35 2.54) (size 2.2 2.2) (drill 1.5) (layers "*.Cu" "*.Mask") (remove_unused_layers no) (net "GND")))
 (gr_rect (start 116.009418 47.014967) (end 180 132.426494) (stroke (width 0.05) (type default)) (fill no) (layer "Edge.Cuts"))
 (segment (start 130.54 61.84) (end 141 51.38) (width 0.2) (layer "B.Cu") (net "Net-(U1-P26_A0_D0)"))
 (segment (start 130.54 74.92) (end 130.54 61.84) (width 0.2) (layer "B.Cu") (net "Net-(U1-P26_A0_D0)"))
 (segment (start 140.165 53.92) (end 142.062 55.817) (width 0.2) (layer "F.Cu") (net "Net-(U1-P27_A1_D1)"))
 (segment (start 142.062 55.817) (end 142.062 59.439895) (width 0.2) (layer "F.Cu") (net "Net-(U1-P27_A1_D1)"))
 (segment (start 141.439895 60.062) (end 138.909786 60.062) (width 0.2) (layer "F.Cu") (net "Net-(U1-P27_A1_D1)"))
 (segment (start 142.062 59.439895) (end 141.439895 60.062) (width 0.2) (layer "F.Cu") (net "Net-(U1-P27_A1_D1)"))
 (segment (start 138.649 86.811) (end 130.54 94.92) (width 0.2) (layer "F.Cu") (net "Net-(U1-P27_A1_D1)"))
 (segment (start 138.649 60.322786) (end 138.649 86.811) (width 0.2) (layer "F.Cu") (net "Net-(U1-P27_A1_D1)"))
 (segment (start 138.909786 60.062) (end 138.649 60.322786) (width 0.2) (layer "F.Cu") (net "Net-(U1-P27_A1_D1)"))
 (segment (start 121.72 74.905) (end 140.165 56.46) (width 0.2) (layer "F.Cu") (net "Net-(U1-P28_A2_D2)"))
 (segment (start 128.709899 114.92) (end 124.769899 118.86) (width 0.2) (layer "F.Cu") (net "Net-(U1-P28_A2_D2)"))
 (segment (start 130.54 114.92) (end 128.709899 114.92) (width 0.2) (layer "F.Cu") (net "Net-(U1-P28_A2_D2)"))
 (segment (start 121.72 116.969899) (end 121.72 74.905) (width 0.2) (layer "F.Cu") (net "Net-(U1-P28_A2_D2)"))
 (segment (start 124.769899 118.86) (end 123.610101 118.86) (width 0.2) (layer "F.Cu") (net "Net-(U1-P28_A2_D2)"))
 (segment (start 123.610101 118.86) (end 121.72 116.969899) (width 0.2) (layer "F.Cu") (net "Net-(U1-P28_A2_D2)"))
 (segment (start 150.54 74.92) (end 150.54 68.54) (width 0.2) (layer "B.Cu") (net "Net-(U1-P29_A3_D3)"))
 (segment (start 150.54 68.54) (end 141 59) (width 0.2) (layer "B.Cu") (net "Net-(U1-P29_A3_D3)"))
 (segment (start 149.14 77.14) (end 149.14 69.68) (width 0.2) (layer "B.Cu") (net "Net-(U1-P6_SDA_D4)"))
 (segment (start 149.14 69.68) (end 141 61.54) (width 0.2) (layer "B.Cu") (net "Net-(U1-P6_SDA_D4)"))
 (segment (start 150.54 94.92) (end 150.54 78.54) (width 0.2) (layer "B.Cu") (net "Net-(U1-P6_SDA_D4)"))
 (segment (start 150.54 78.54) (end 149.14 77.14) (width 0.2) (layer "B.Cu") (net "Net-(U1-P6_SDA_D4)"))
 (segment (start 171.86 95.579899) (end 171.94 95.499899) (width 0.2) (layer "F.Cu") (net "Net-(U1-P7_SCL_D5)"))
 (segment (start 171.94 94.340101) (end 171.079899 93.48) (width 0.2) (layer "F.Cu") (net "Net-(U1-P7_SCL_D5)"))
 (segment (start 169.880101 116.32) (end 171.039899 116.32) (width 0.2) (layer "F.Cu") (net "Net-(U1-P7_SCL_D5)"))
 (segment (start 171.9 75.499899) (end 171.9 74.047786) (width 0.2) (layer "F.Cu") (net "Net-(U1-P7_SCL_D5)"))
 (segment (start 168.480101 114.92) (end 169.880101 116.32) (width 0.2) (layer "F.Cu") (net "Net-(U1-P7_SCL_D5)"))
 (segment (start 150.54 114.92) (end 168.480101 114.92) (width 0.2) (layer "F.Cu") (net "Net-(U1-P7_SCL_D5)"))
 (segment (start 171.039899 116.32) (end 171.86 115.499899) (width 0.2) (layer "F.Cu") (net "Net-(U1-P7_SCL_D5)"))
 (segment (start 171.079899 93.48) (end 171.079899 76.32) (width 0.2) (layer "F.Cu") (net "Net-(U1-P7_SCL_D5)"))
 (segment (start 171.94 95.499899) (end 171.94 94.340101) (width 0.2) (layer "F.Cu") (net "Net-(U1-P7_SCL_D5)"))
 (segment (start 171.9 74.047786) (end 158.330214 60.478) (width 0.2) (layer "F.Cu") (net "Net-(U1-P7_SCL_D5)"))
 (segment (start 171.86 115.499899) (end 171.86 95.579899) (width 0.2) (layer "F.Cu") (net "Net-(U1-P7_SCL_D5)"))
 (segment (start 144.602 60.478) (end 141 64.08) (width 0.2) (layer "F.Cu") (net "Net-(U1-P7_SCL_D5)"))
 (segment (start 158.330214 60.478) (end 144.602 60.478) (width 0.2) (layer "F.Cu") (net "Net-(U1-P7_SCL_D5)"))
 (segment (start 171.079899 76.32) (end 171.9 75.499899) (width 0.2) (layer "F.Cu") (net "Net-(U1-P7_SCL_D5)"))
 (segment (start 145.002 62.618) (end 141 66.62) (width 0.2) (layer "F.Cu") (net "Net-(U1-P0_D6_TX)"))
 (segment (start 159.753634 62.618) (end 145.002 62.618) (width 0.2) (layer "F.Cu") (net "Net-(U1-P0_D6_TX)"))
 (segment (start 170.5 73.364366) (end 159.753634 62.618) (width 0.2) (layer "F.Cu") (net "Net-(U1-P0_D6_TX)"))
 (segment (start 170.5 74.92) (end 170.5 73.364366) (width 0.2) (layer "F.Cu") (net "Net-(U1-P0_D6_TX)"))
 (segment (start 158.591 63.278786) (end 158.330214 63.018) (width 0.2) (layer "F.Cu") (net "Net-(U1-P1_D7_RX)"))
 (segment (start 158.330214 63.018) (end 155.800105 63.018) (width 0.2) (layer "F.Cu") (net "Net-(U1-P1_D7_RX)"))
 (segment (start 155.178 64.723) (end 157.075 66.62) (width 0.2) (layer "F.Cu") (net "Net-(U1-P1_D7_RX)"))
 (segment (start 155.800105 63.018) (end 155.178 63.640105) (width 0.2) (layer "F.Cu") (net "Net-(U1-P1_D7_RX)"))
 (segment (start 170.54 76.979314) (end 158.591 65.030314) (width 0.2) (layer "F.Cu") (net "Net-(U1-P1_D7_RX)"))
 (segment (start 158.591 65.030314) (end 158.591 63.278786) (width 0.2) (layer "F.Cu") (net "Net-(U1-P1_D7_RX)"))
 (segment (start 155.178 63.640105) (end 155.178 64.723) (width 0.2) (layer "F.Cu") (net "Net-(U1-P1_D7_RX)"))
 (segment (start 170.54 94.92) (end 170.54 76.979314) (width 0.2) (layer "F.Cu") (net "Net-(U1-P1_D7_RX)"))
 (segment (start 165.55 72.555) (end 157.075 64.08) (width 0.2) (layer "F.Cu") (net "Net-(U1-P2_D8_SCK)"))
 (segment (start 170.46 98.46) (end 165.55 93.55) (width 0.2) (layer "F.Cu") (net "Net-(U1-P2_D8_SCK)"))
 (segment (start 165.55 93.55) (end 165.55 72.555) (width 0.2) (layer "F.Cu") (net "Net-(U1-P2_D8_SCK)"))
 (segment (start 170.46 114.92) (end 170.46 98.46) (width 0.2) (layer "F.Cu") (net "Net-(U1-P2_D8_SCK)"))
 (segment (start 124.19 77.46) (end 124.19 117.46) (width 0.2) (layer "F.Cu") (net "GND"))
 (segment (start 164.15 77.46) (end 144.19 77.46) (width 0.2) (layer "F.Cu") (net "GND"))
 (segment (start 144.19 77.46) (end 144.19 117.46) (width 0.2) (layer "F.Cu") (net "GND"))
 (segment (start 124.19 97.46) (end 164.19 97.46) (width 0.2) (layer "F.Cu") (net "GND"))
 (segment (start 164.11 117.46) (end 144.19 117.46) (width 0.2) (layer "F.Cu") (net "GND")))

